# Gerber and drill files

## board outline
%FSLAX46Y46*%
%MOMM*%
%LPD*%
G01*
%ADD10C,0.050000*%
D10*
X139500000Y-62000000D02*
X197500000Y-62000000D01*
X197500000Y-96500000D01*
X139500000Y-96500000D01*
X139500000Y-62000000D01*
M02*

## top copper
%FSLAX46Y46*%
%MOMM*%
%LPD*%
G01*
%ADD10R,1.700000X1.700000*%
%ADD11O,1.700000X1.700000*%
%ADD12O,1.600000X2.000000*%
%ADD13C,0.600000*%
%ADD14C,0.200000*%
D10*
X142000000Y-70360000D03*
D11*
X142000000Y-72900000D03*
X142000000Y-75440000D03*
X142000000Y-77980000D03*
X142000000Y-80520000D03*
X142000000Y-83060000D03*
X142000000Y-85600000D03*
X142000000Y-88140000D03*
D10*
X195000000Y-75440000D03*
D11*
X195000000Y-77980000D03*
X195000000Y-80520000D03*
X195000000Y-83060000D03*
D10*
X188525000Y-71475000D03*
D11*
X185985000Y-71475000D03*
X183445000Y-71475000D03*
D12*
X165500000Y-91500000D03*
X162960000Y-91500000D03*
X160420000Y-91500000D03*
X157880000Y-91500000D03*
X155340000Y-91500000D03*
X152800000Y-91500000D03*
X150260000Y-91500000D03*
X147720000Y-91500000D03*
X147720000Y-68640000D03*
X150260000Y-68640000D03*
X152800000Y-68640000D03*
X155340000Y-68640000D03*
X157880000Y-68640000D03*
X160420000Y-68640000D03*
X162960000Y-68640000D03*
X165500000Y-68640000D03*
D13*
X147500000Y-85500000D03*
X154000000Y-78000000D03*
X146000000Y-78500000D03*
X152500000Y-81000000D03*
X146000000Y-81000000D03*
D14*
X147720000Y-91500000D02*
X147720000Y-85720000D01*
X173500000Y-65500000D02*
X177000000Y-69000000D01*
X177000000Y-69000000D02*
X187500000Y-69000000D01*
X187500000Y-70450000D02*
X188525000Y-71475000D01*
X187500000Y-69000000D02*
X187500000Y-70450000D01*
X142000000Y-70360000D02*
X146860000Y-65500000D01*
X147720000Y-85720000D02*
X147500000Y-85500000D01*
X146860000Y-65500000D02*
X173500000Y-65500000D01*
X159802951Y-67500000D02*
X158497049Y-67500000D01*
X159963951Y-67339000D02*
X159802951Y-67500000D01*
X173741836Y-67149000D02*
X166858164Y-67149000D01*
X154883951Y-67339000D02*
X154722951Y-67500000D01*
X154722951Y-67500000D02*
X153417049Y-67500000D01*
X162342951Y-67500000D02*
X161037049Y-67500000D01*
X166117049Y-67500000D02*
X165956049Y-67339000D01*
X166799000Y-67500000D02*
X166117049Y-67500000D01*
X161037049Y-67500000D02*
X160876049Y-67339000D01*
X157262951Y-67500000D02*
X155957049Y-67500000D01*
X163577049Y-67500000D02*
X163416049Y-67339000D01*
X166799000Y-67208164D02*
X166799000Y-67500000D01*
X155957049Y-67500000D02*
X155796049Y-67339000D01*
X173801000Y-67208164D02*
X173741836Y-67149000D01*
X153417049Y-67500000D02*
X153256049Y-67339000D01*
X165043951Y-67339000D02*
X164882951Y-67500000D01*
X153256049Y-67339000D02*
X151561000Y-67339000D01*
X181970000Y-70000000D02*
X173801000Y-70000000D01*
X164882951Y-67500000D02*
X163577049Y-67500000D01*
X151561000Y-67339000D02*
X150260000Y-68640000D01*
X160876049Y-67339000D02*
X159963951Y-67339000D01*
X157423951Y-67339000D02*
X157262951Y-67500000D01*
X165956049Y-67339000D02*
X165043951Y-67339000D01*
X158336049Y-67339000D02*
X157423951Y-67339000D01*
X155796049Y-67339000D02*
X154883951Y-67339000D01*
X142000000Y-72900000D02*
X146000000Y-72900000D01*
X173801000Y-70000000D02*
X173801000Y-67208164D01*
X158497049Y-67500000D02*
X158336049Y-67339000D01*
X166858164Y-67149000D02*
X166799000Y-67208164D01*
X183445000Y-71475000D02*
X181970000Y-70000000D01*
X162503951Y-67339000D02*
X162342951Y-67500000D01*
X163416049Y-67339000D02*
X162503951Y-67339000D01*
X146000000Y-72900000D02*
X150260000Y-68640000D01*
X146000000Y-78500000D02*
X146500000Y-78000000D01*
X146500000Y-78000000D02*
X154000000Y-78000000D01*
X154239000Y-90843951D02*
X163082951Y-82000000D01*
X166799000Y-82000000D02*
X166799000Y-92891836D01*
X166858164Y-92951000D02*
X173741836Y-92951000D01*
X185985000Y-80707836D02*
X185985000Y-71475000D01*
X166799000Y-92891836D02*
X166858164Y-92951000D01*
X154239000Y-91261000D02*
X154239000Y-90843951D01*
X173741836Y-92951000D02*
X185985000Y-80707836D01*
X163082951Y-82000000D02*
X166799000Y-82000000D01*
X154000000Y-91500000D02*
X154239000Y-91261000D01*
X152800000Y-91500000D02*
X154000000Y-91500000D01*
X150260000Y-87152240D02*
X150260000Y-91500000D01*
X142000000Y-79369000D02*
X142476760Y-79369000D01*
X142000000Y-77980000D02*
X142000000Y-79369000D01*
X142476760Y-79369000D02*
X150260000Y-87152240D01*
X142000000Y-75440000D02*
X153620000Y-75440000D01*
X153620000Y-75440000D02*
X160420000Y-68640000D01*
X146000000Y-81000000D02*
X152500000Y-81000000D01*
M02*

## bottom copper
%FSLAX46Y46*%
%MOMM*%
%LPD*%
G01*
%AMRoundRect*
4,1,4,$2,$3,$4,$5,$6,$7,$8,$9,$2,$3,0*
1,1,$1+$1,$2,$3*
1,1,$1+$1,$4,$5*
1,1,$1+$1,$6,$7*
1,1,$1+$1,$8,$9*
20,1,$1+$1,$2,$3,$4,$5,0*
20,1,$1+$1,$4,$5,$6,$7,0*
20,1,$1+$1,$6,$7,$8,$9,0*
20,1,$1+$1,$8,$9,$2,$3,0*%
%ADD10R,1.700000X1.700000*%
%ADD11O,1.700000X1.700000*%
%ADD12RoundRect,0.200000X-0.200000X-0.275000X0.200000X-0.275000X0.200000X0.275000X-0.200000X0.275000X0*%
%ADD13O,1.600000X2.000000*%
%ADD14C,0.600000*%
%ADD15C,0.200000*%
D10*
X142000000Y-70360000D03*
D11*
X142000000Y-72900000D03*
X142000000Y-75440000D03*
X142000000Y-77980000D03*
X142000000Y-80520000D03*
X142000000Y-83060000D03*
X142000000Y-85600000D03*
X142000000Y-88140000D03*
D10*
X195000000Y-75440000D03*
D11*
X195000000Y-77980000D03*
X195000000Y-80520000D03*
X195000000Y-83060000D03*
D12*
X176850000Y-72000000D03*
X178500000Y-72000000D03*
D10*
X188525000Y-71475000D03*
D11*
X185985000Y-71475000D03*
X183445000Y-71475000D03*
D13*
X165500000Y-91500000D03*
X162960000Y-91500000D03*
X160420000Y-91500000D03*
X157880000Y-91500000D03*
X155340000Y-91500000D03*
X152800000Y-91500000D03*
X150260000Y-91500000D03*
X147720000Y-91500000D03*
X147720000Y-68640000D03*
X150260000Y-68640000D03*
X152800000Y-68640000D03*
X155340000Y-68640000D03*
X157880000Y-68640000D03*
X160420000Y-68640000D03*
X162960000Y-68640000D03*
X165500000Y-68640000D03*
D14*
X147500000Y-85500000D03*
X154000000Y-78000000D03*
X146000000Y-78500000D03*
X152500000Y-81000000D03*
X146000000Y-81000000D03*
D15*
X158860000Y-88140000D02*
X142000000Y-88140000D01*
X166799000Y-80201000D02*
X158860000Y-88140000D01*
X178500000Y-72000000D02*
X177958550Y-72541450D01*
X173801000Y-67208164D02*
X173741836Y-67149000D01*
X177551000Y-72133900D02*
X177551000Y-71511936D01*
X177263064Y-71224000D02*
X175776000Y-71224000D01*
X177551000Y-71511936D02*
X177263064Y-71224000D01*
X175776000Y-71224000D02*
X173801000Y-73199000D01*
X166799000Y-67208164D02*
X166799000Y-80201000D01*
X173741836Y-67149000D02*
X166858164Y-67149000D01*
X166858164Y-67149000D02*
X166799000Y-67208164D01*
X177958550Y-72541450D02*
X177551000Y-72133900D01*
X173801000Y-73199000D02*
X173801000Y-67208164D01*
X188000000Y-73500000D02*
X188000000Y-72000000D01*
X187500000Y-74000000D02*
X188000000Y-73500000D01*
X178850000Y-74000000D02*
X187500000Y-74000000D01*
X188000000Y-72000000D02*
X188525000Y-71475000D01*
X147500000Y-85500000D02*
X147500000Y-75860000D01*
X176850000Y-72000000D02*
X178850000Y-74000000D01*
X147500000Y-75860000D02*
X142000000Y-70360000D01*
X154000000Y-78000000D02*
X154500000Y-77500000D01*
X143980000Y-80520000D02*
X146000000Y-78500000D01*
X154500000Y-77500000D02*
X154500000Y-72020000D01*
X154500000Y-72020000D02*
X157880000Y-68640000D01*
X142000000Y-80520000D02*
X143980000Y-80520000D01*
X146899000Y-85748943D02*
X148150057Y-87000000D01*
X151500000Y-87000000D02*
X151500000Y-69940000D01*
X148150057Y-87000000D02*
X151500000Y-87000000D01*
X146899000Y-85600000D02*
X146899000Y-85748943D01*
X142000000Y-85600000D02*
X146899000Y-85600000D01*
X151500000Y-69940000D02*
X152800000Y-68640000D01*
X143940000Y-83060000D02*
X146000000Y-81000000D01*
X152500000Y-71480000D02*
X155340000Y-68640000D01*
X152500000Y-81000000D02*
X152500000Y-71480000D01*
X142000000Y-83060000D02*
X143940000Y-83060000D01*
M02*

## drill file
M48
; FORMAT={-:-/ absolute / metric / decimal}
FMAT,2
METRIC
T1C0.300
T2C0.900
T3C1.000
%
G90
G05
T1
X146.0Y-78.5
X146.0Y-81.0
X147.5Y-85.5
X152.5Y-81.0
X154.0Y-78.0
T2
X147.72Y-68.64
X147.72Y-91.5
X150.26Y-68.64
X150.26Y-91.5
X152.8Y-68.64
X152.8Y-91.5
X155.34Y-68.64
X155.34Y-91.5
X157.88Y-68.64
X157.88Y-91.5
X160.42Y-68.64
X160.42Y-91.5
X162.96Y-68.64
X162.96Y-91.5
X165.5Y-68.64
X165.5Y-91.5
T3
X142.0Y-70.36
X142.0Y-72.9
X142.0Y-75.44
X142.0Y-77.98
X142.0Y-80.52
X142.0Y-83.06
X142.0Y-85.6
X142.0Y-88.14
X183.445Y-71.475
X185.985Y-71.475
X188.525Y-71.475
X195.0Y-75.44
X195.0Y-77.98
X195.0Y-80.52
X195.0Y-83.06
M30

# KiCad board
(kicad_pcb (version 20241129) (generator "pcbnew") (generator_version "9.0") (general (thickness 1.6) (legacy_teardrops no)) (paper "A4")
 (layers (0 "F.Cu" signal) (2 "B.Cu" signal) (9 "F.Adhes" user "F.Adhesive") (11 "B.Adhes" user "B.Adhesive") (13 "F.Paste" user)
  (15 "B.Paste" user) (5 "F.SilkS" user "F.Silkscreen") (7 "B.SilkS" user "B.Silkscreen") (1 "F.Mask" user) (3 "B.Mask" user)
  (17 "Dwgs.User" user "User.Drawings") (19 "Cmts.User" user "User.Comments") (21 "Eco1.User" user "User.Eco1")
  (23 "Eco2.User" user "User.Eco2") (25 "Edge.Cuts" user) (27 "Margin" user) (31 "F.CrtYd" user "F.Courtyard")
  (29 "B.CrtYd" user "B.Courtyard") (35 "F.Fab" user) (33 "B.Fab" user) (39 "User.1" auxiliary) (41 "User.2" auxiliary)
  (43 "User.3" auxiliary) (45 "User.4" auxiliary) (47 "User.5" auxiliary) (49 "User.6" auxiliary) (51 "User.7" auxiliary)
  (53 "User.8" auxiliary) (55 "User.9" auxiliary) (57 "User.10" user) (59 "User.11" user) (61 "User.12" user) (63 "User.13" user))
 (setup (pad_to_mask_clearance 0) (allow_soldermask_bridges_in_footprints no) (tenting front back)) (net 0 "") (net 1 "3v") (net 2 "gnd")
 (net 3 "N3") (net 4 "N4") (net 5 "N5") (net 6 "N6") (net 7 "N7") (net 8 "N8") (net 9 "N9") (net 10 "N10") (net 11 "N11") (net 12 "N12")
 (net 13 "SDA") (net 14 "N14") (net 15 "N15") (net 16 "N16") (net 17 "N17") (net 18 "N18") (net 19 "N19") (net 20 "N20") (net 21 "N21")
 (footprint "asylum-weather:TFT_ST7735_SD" (layer "F.Cu") (at 162 79)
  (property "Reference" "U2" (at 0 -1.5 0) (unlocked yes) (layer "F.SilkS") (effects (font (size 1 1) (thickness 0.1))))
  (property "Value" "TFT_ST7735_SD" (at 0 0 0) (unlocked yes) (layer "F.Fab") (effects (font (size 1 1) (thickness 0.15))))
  (pad "1" thru_hole rect (at -20 -8.64) (size 1.7 1.7) (drill 1) (layers "*.Cu" "*.Mask") (remove_unused_layers no) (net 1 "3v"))
  (pad "2" thru_hole oval (at -20 -6.1) (size 1.7 1.7) (drill 1) (layers "*.Cu" "*.Mask") (remove_unused_layers no) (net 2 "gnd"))
  (pad "3" thru_hole oval (at -20 -3.56) (size 1.7 1.7) (drill 1) (layers "*.Cu" "*.Mask") (remove_unused_layers no) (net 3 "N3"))
  (pad "4" thru_hole oval (at -20 -1.02) (size 1.7 1.7) (drill 1) (layers "*.Cu" "*.Mask") (remove_unused_layers no) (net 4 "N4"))
  (pad "5" thru_hole oval (at -20 1.52) (size 1.7 1.7) (drill 1) (layers "*.Cu" "*.Mask") (remove_unused_layers no) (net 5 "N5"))
  (pad "6" thru_hole oval (at -20 4.06) (size 1.7 1.7) (drill 1) (layers "*.Cu" "*.Mask") (remove_unused_layers no) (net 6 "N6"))
  (pad "7" thru_hole oval (at -20 6.6) (size 1.7 1.7) (drill 1) (layers "*.Cu" "*.Mask") (remove_unused_layers no) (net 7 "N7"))
  (pad "8" thru_hole oval (at -20 9.14) (size 1.7 1.7) (drill 1) (layers "*.Cu" "*.Mask") (remove_unused_layers no) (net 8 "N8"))
  (pad "9" thru_hole rect (at 33 -3.56) (size 1.7 1.7) (drill 1) (layers "*.Cu" "*.Mask") (remove_unused_layers no) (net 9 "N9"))
  (pad "10" thru_hole oval (at 33 -1.02) (size 1.7 1.7) (drill 1) (layers "*.Cu" "*.Mask") (remove_unused_layers no) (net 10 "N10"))
  (pad "11" thru_hole oval (at 33 1.52) (size 1.7 1.7) (drill 1) (layers "*.Cu" "*.Mask") (remove_unused_layers no) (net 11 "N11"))
  (pad "12" thru_hole oval (at 33 4.06) (size 1.7 1.7) (drill 1) (layers "*.Cu" "*.Mask") (remove_unused_layers no) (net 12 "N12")))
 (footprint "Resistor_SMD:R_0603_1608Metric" (layer "B.Cu") (at 177.675 72)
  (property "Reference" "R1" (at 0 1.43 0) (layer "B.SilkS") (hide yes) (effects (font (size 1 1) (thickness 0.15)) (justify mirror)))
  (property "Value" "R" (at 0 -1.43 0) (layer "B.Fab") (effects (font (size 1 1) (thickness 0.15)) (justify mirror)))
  (pad "1" smd roundrect (at -0.825 0) (size 0.8 0.95) (layers "B.Cu" "B.Mask" "B.Paste") (roundrect_rratio 0.25) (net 1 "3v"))
  (pad "2" smd roundrect (at 0.825 0) (size 0.8 0.95) (layers "B.Cu" "B.Mask" "B.Paste") (roundrect_rratio 0.25) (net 8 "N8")))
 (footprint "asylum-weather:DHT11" (layer "B.Cu") (at 188.525 71.475 90)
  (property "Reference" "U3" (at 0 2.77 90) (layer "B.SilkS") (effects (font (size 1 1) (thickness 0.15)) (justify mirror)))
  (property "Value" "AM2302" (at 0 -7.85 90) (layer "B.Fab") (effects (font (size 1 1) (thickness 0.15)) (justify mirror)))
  (pad "1" thru_hole rect (at 0 0 90) (size 1.7 1.7) (drill 1) (layers "F&B.Cu" "*.Mask") (remove_unused_layers no) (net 1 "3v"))
  (pad "2" thru_hole oval (at 0 -2.54 90) (size 1.7 1.7) (drill 1) (layers "F&B.Cu" "*.Mask") (remove_unused_layers no) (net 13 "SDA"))
  (pad "3" thru_hole oval (at 0 -5.08 90) (size 1.7 1.7) (drill 1) (layers "F&B.Cu" "*.Mask") (remove_unused_layers no) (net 2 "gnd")))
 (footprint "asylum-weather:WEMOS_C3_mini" (layer "B.Cu") (at 158 80.07 90)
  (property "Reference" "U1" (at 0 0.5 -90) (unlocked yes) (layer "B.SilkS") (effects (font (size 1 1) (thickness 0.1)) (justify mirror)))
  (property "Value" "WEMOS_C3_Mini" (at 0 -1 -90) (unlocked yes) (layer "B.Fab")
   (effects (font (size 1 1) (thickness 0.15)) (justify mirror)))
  (pad "1" thru_hole oval (at -11.43 7.5 90) (size 2 1.6) (drill 0.9) (layers "F&B.Cu" "*.Mask") (remove_unused_layers no) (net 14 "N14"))
  (pad "2" thru_hole oval (at -11.43 4.96 90) (size 2 1.6) (drill 0.9) (layers "F&B.Cu" "*.Mask") (remove_unused_layers no) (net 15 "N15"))
  (pad "3" thru_hole oval (at -11.43 2.42 90) (size 2 1.6) (drill 0.9) (layers "F&B.Cu" "*.Mask") (remove_unused_layers no) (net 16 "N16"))
  (pad "4" thru_hole oval (at -11.43 -0.12 90) (size 2 1.6) (drill 0.9) (layers "F&B.Cu" "*.Mask") (remove_unused_layers no) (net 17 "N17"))
  (pad "5" thru_hole oval (at -11.43 -2.66 90) (size 2 1.6) (drill 0.9) (layers "F&B.Cu" "*.Mask") (remove_unused_layers no) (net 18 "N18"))
  (pad "6" thru_hole oval (at -11.43 -5.2 90) (size 2 1.6) (drill 0.9) (layers "F&B.Cu" "*.Mask") (remove_unused_layers no) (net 13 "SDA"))
  (pad "7" thru_hole oval (at -11.43 -7.74 90) (size 2 1.6) (drill 0.9) (layers "F&B.Cu" "*.Mask") (remove_unused_layers no) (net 4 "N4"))
  (pad "8" thru_hole oval (at -11.43 -10.28 90) (size 2 1.6) (drill 0.9) (layers "F&B.Cu" "*.Mask") (remove_unused_layers no) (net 1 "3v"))
  (pad "9" thru_hole oval (at 11.43 -10.28 90) (size 2 1.6) (drill 0.9) (layers "F&B.Cu" "*.Mask") (remove_unused_layers no) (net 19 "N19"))
  (pad "10" thru_hole oval (at 11.43 -7.74 90) (size 2 1.6) (drill 0.9) (layers "F&B.Cu" "*.Mask") (remove_unused_layers no) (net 2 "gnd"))
  (pad "11" thru_hole oval (at 11.43 -5.2 90) (size 2 1.6) (drill 0.9) (layers "F&B.Cu" "*.Mask") (remove_unused_layers no) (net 7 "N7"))
  (pad "12" thru_hole oval (at 11.43 -2.66 90) (size 2 1.6) (drill 0.9) (layers "F&B.Cu" "*.Mask") (remove_unused_layers no) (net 6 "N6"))
  (pad "13" thru_hole oval (at 11.43 -0.12 90) (size 2 1.6) (drill 0.9) (layers "F&B.Cu" "*.Mask") (remove_unused_layers no) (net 5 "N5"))
  (pad "14" thru_hole oval (at 11.43 2.42 90) (size 2 1.6) (drill 0.9) (layers "F&B.Cu" "*.Mask") (remove_unused_layers no) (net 3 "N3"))
  (pad "15" thru_hole oval (at 11.43 4.96 90) (size 2 1.6) (drill 0.9) (layers "F&B.Cu" "*.Mask") (remove_unused_layers no) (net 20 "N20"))
  (pad "16" thru_hole oval (at 11.43 7.5 90) (size 2 1.6) (drill 0.9) (layers "F&B.Cu" "*.Mask") (remove_unused_layers no) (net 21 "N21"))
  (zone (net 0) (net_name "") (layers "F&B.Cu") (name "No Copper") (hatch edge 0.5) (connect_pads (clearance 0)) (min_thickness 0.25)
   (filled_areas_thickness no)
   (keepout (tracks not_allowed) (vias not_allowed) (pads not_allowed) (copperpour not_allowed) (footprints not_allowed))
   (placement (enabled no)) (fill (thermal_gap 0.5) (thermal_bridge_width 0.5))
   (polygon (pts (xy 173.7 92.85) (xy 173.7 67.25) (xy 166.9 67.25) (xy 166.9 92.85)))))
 (gr_rect (start 139.5 62) (end 197.5 96.5) (stroke (width 0.05) (type default)) (fill no) (layer "Edge.Cuts"))
 (segment (start 158.86 88.14) (end 142 88.14) (width 0.2) (layer "B.Cu") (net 8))
 (segment (start 166.799 80.201) (end 158.86 88.14) (width 0.2) (layer "B.Cu") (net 8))
 (segment (start 178.5 72) (end 177.95855 72.54145) (width 0.2) (layer "B.Cu") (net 8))
 (segment (start 173.801 67.208164) (end 173.741836 67.149) (width 0.2) (layer "B.Cu") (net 8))
 (segment (start 177.551 72.1339) (end 177.551 71.511936) (width 0.2) (layer "B.Cu") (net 8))
 (segment (start 177.263064 71.224) (end 175.776 71.224) (width 0.2) (layer "B.Cu") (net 8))
 (segment (start 177.551 71.511936) (end 177.263064 71.224) (width 0.2) (layer "B.Cu") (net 8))
 (segment (start 175.776 71.224) (end 173.801 73.199) (width 0.2) (layer "B.Cu") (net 8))
 (segment (start 166.799 67.208164) (end 166.799 80.201) (width 0.2) (layer "B.Cu") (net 8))
 (segment (start 173.741836 67.149) (end 166.858164 67.149) (width 0.2) (layer "B.Cu") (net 8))
 (segment (start 166.858164 67.149) (end 166.799 67.208164) (width 0.2) (layer "B.Cu") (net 8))
 (segment (start 177.95855 72.54145) (end 177.551 72.1339) (width 0.2) (layer "B.Cu") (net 8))
 (segment (start 173.801 73.199) (end 173.801 67.208164) (width 0.2) (layer "B.Cu") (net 8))
 (segment (start 147.72 91.5) (end 147.72 85.72) (width 0.2) (layer "F.Cu") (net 1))
 (segment (start 173.5 65.5) (end 177 69) (width 0.2) (layer "F.Cu") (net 1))
 (segment (start 177 69) (end 187.5 69) (width 0.2) (layer "F.Cu") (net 1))
 (segment (start 187.5 70.45) (end 188.525 71.475) (width 0.2) (layer "F.Cu") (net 1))
 (segment (start 187.5 69) (end 187.5 70.45) (width 0.2) (layer "F.Cu") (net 1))
 (segment (start 142 70.36) (end 146.86 65.5) (width 0.2) (layer "F.Cu") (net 1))
 (segment (start 147.72 85.72) (end 147.5 85.5) (width 0.2) (layer "F.Cu") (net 1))
 (segment (start 146.86 65.5) (end 173.5 65.5) (width 0.2) (layer "F.Cu") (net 1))
 (via (at 147.5 85.5) (size 0.6) (drill 0.3) (layers "F.Cu" "B.Cu") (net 1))
 (segment (start 188 73.5) (end 188 72) (width 0.2) (layer "B.Cu") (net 1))
 (segment (start 187.5 74) (end 188 73.5) (width 0.2) (layer "B.Cu") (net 1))
 (segment (start 178.85 74) (end 187.5 74) (width 0.2) (layer "B.Cu") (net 1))
 (segment (start 188 72) (end 188.525 71.475) (width 0.2) (layer "B.Cu") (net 1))
 (segment (start 147.5 85.5) (end 147.5 75.86) (width 0.2) (layer "B.Cu") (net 1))
 (segment (start 176.85 72) (end 178.85 74) (width 0.2) (layer "B.Cu") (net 1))
 (segment (start 147.5 75.86) (end 142 70.36) (width 0.2) (layer "B.Cu") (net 1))
 (segment (start 159.802951 67.5) (end 158.497049 67.5) (width 0.2) (layer "F.Cu") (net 2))
 (segment (start 159.963951 67.339) (end 159.802951 67.5) (width 0.2) (layer "F.Cu") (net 2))
 (segment (start 173.741836 67.149) (end 166.858164 67.149) (width 0.2) (layer "F.Cu") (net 2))
 (segment (start 154.883951 67.339) (end 154.722951 67.5) (width 0.2) (layer "F.Cu") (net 2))
 (segment (start 154.722951 67.5) (end 153.417049 67.5) (width 0.2) (layer "F.Cu") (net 2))
 (segment (start 162.342951 67.5) (end 161.037049 67.5) (width 0.2) (layer "F.Cu") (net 2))
 (segment (start 166.117049 67.5) (end 165.956049 67.339) (width 0.2) (layer "F.Cu") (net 2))
 (segment (start 166.799 67.5) (end 166.117049 67.5) (width 0.2) (layer "F.Cu") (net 2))
 (segment (start 161.037049 67.5) (end 160.876049 67.339) (width 0.2) (layer "F.Cu") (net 2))
 (segment (start 157.262951 67.5) (end 155.957049 67.5) (width 0.2) (layer "F.Cu") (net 2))
 (segment (start 163.577049 67.5) (end 163.416049 67.339) (width 0.2) (layer "F.Cu") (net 2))
 (segment (start 166.799 67.208164) (end 166.799 67.5) (width 0.2) (layer "F.Cu") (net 2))
 (segment (start 155.957049 67.5) (end 155.796049 67.339) (width 0.2) (layer "F.Cu") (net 2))
 (segment (start 173.801 67.208164) (end 173.741836 67.149) (width 0.2) (layer "F.Cu") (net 2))
 (segment (start 153.417049 67.5) (end 153.256049 67.339) (width 0.2) (layer "F.Cu") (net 2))
 (segment (start 165.043951 67.339) (end 164.882951 67.5) (width 0.2) (layer "F.Cu") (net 2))
 (segment (start 153.256049 67.339) (end 151.561 67.339) (width 0.2) (layer "F.Cu") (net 2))
 (segment (start 181.97 70) (end 173.801 70) (width 0.2) (layer "F.Cu") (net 2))
 (segment (start 164.882951 67.5) (end 163.577049 67.5) (width 0.2) (layer "F.Cu") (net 2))
 (segment (start 151.561 67.339) (end 150.26 68.64) (width 0.2) (layer "F.Cu") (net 2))
 (segment (start 160.876049 67.339) (end 159.963951 67.339) (width 0.2) (layer "F.Cu") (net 2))
 (segment (start 157.423951 67.339) (end 157.262951 67.5) (width 0.2) (layer "F.Cu") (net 2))
 (segment (start 165.956049 67.339) (end 165.043951 67.339) (width 0.2) (layer "F.Cu") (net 2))
 (segment (start 158.336049 67.339) (end 157.423951 67.339) (width 0.2) (layer "F.Cu") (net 2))
 (segment (start 155.796049 67.339) (end 154.883951 67.339) (width 0.2) (layer "F.Cu") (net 2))
 (segment (start 142 72.9) (end 146 72.9) (width 0.2) (layer "F.Cu") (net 2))
 (segment (start 173.801 70) (end 173.801 67.208164) (width 0.2) (layer "F.Cu") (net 2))
 (segment (start 158.497049 67.5) (end 158.336049 67.339) (width 0.2) (layer "F.Cu") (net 2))
 (segment (start 166.858164 67.149) (end 166.799 67.208164) (width 0.2) (layer "F.Cu") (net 2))
 (segment (start 183.445 71.475) (end 181.97 70) (width 0.2) (layer "F.Cu") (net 2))
 (segment (start 162.503951 67.339) (end 162.342951 67.5) (width 0.2) (layer "F.Cu") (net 2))
 (segment (start 163.416049 67.339) (end 162.503951 67.339) (width 0.2) (layer "F.Cu") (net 2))
 (segment (start 146 72.9) (end 150.26 68.64) (width 0.2) (layer "F.Cu") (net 2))
 (segment (start 146 78.5) (end 146.5 78) (width 0.2) (layer "F.Cu") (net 5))
 (segment (start 146.5 78) (end 154 78) (width 0.2) (layer "F.Cu") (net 5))
 (via (at 154 78) (size 0.6) (drill 0.3) (layers "F.Cu" "B.Cu") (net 5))
 (via (at 146 78.5) (size 0.6) (drill 0.3) (layers "F.Cu" "B.Cu") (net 5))
 (segment (start 154 78) (end 154.5 77.5) (width 0.2) (layer "B.Cu") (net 5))
 (segment (start 143.98 80.52) (end 146 78.5) (width 0.2) (layer "B.Cu") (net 5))
 (segment (start 154.5 77.5) (end 154.5 72.02) (width 0.2) (layer "B.Cu") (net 5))
 (segment (start 154.5 72.02) (end 157.88 68.64) (width 0.2) (layer "B.Cu") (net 5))
 (segment (start 142 80.52) (end 143.98 80.52) (width 0.2) (layer "B.Cu") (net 5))
 (segment (start 154.239 90.843951) (end 163.082951 82) (width 0.2) (layer "F.Cu") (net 13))
 (segment (start 166.799 82) (end 166.799 92.891836) (width 0.2) (layer "F.Cu") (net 13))
 (segment (start 166.858164 92.951) (end 173.741836 92.951) (width 0.2) (layer "F.Cu") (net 13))
 (segment (start 185.985 80.707836) (end 185.985 71.475) (width 0.2) (layer "F.Cu") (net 13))
 (segment (start 166.799 92.891836) (end 166.858164 92.951) (width 0.2) (layer "F.Cu") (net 13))
 (segment (start 154.239 91.261) (end 154.239 90.843951) (width 0.2) (layer "F.Cu") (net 13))
 (segment (start 173.741836 92.951) (end 185.985 80.707836) (width 0.2) (layer "F.Cu") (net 13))
 (segment (start 163.082951 82) (end 166.799 82) (width 0.2) (layer "F.Cu") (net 13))
 (segment (start 154 91.5) (end 154.239 91.261) (width 0.2) (layer "F.Cu") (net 13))
 (segment (start 152.8 91.5) (end 154 91.5) (width 0.2) (layer "F.Cu") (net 13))
 (segment (start 150.26 87.15224) (end 150.26 91.5) (width 0.2) (layer "F.Cu") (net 4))
 (segment (start 142 79.369) (end 142.47676 79.369) (width 0.2) (layer "F.Cu") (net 4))
 (segment (start 142 77.98) (end 142 79.369) (width 0.2) (layer "F.Cu") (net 4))
 (segment (start 142.47676 79.369) (end 150.26 87.15224) (width 0.2) (layer "F.Cu") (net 4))
 (segment (start 146.899 85.748943) (end 148.150057 87) (width 0.2) (layer "B.Cu") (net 7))
 (segment (start 151.5 87) (end 151.5 69.94) (width 0.2) (layer "B.Cu") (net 7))
 (segment (start 148.150057 87) (end 151.5 87) (width 0.2) (layer "B.Cu") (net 7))
 (segment (start 146.899 85.6) (end 146.899 85.748943) (width 0.2) (layer "B.Cu") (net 7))
 (segment (start 142 85.6) (end 146.899 85.6) (width 0.2) (layer "B.Cu") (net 7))
 (segment (start 151.5 69.94) (end 152.8 68.64) (width 0.2) (layer "B.Cu") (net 7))
 (segment (start 142 75.44) (end 153.62 75.44) (width 0.2) (layer "F.Cu") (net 3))
 (segment (start 153.62 75.44) (end 160.42 68.64) (width 0.2) (layer "F.Cu") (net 3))
 (segment (start 146 81) (end 152.5 81) (width 0.2) (layer "F.Cu") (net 6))
 (via (at 152.5 81) (size 0.6) (drill 0.3) (layers "F.Cu" "B.Cu") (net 6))
 (via (at 146 81) (size 0.6) (drill 0.3) (layers "F.Cu" "B.Cu") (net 6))
 (segment (start 143.94 83.06) (end 146 81) (width 0.2) (layer "B.Cu") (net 6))
 (segment (start 152.5 71.48) (end 155.34 68.64) (width 0.2) (layer "B.Cu") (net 6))
 (segment (start 152.5 81) (end 152.5 71.48) (width 0.2) (layer "B.Cu") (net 6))
 (segment (start 142 83.06) (end 143.94 83.06) (width 0.2) (layer "B.Cu") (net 6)))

